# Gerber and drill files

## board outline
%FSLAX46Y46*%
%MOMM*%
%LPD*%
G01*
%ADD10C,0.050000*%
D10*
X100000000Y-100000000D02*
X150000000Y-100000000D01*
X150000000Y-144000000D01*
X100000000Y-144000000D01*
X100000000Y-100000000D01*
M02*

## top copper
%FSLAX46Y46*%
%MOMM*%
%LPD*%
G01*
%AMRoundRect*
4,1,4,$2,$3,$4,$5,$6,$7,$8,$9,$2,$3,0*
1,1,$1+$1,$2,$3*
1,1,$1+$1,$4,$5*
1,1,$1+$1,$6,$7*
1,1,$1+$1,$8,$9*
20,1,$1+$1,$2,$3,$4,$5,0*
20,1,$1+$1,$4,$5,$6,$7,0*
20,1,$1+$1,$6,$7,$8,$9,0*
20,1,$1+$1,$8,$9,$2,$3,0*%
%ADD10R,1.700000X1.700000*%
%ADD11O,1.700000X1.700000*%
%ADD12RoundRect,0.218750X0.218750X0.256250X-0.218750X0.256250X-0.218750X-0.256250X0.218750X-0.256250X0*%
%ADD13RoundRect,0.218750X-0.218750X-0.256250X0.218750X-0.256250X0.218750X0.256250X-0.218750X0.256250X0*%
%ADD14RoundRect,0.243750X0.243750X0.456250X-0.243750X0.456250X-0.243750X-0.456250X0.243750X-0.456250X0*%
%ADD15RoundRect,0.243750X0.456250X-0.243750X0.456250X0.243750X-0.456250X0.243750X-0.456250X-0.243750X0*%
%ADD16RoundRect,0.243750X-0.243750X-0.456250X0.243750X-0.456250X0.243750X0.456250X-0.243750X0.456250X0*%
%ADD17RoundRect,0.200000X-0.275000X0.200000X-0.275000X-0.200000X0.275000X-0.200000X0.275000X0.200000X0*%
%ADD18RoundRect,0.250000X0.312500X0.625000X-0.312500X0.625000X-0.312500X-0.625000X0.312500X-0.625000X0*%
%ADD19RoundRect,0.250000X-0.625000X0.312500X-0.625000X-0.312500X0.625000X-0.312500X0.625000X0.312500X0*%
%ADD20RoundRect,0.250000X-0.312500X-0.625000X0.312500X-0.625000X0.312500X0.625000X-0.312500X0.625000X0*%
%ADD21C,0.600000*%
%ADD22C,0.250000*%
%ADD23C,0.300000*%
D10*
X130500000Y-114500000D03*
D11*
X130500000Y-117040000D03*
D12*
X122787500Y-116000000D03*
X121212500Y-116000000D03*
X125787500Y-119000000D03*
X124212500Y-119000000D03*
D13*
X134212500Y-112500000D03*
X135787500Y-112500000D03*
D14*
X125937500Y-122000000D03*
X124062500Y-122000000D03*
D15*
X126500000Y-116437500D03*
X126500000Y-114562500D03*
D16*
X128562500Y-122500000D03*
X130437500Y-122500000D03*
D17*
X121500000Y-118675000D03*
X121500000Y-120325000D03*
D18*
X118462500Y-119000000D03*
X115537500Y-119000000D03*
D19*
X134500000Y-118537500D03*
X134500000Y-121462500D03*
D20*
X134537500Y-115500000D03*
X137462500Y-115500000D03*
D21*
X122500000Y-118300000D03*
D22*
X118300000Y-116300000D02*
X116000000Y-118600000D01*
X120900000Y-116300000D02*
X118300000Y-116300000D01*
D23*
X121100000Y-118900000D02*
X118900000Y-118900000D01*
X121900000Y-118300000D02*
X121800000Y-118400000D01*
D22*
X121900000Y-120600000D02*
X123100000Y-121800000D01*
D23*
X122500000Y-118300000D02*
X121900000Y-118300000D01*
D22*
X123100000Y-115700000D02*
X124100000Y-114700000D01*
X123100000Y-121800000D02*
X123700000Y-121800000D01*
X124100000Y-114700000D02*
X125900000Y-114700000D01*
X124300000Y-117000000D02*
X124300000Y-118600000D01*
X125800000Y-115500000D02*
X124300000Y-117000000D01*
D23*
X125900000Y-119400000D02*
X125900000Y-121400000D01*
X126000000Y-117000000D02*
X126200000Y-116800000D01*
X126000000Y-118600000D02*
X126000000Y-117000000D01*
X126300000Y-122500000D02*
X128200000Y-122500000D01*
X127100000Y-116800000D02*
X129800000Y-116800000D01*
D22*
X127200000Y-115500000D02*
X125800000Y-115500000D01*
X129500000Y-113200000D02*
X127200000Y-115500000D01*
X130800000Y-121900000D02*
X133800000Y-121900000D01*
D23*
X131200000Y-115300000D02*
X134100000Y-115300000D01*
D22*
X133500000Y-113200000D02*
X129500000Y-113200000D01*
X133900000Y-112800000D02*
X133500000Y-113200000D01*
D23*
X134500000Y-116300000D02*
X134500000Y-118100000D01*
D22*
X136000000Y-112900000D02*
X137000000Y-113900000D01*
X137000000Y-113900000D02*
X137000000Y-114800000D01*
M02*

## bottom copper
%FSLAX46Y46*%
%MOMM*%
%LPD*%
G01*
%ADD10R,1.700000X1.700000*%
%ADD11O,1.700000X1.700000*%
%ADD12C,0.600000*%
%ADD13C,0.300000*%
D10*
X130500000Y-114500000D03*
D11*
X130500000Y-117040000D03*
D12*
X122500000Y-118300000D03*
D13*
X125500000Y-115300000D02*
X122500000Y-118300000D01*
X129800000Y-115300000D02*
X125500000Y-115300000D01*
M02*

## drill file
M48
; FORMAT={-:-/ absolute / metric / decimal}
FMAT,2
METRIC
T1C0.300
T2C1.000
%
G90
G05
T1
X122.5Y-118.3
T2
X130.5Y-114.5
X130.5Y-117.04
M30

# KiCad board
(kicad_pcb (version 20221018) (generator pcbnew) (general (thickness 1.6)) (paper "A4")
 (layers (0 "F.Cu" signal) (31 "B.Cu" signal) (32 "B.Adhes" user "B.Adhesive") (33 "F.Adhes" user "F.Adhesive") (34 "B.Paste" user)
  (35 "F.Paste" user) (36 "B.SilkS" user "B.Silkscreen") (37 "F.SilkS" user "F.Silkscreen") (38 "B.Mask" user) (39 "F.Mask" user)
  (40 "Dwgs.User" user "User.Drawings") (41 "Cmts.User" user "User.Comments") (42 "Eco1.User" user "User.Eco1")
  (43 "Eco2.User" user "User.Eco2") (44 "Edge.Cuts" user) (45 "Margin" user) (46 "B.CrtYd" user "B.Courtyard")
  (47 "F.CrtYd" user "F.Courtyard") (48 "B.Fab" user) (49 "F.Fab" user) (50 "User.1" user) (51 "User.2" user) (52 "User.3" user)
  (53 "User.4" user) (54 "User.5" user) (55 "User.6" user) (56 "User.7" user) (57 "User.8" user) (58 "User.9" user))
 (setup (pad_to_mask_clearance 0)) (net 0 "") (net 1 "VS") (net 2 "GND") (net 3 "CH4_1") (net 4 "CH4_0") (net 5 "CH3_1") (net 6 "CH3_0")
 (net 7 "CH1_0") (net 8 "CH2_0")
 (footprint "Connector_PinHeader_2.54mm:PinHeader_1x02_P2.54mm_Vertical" (layer "F.Cu") (at 130.5 114.5)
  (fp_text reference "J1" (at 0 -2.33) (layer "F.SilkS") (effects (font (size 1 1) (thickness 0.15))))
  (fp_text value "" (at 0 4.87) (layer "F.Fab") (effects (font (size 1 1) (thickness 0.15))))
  (pad "1" thru_hole rect (at 0 0) (size 1.7 1.7) (drill 1) (layers "*.Cu" "*.Mask") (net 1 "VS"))
  (pad "2" thru_hole oval (at 0 2.54) (size 1.7 1.7) (drill 1) (layers "*.Cu" "*.Mask") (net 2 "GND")))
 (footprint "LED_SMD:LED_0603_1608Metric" (layer "F.Cu") (at 122 116 180)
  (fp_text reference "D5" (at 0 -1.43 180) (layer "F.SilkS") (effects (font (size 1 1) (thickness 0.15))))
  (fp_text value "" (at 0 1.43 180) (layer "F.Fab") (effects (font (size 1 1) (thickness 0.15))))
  (pad "1" smd roundrect (at -0.7875 0 180) (size 0.875 0.95) (layers "F.Cu" "F.Paste" "F.Mask") (roundrect_rratio 0.25) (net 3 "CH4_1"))
  (pad "2" smd roundrect (at 0.7875 0 180) (size 0.875 0.95) (layers "F.Cu" "F.Paste" "F.Mask") (roundrect_rratio 0.25) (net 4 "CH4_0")))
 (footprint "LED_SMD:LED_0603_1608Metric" (layer "F.Cu") (at 125 119 180)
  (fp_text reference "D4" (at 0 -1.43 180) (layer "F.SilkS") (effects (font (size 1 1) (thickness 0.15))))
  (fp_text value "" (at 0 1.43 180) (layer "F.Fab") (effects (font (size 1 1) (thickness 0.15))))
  (pad "1" smd roundrect (at -0.7875 0 180) (size 0.875 0.95) (layers "F.Cu" "F.Paste" "F.Mask") (roundrect_rratio 0.25) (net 2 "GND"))
  (pad "2" smd roundrect (at 0.7875 0 180) (size 0.875 0.95) (layers "F.Cu" "F.Paste" "F.Mask") (roundrect_rratio 0.25) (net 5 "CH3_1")))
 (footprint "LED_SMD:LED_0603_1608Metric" (layer "F.Cu") (at 135 112.5)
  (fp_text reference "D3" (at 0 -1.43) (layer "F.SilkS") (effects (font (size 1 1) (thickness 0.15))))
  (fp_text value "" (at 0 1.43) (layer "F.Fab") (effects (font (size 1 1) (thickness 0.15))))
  (pad "1" smd roundrect (at -0.7875 0) (size 0.875 0.95) (layers "F.Cu" "F.Paste" "F.Mask") (roundrect_rratio 0.25) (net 5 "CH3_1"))
  (pad "2" smd roundrect (at 0.7875 0) (size 0.875 0.95) (layers "F.Cu" "F.Paste" "F.Mask") (roundrect_rratio 0.25) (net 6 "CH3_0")))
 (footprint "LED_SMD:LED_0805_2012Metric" (layer "F.Cu") (at 125 122 180)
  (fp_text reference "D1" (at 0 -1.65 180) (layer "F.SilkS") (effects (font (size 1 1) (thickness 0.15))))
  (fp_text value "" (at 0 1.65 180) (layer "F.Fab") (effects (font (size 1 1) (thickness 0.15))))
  (pad "1" smd roundrect (at -0.9375 0 180) (size 0.975 1.4) (layers "F.Cu" "F.Paste" "F.Mask") (roundrect_rratio 0.25) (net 2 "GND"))
  (pad "2" smd roundrect (at 0.9375 0 180) (size 0.975 1.4) (layers "F.Cu" "F.Paste" "F.Mask") (roundrect_rratio 0.25) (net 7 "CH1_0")))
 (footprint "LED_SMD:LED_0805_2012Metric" (layer "F.Cu") (at 126.5 115.5 90)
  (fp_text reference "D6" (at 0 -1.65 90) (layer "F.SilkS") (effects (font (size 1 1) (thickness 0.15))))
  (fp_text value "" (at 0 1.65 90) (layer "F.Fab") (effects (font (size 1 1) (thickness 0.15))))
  (pad "1" smd roundrect (at -0.9375 0 90) (size 0.975 1.4) (layers "F.Cu" "F.Paste" "F.Mask") (roundrect_rratio 0.25) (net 2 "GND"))
  (pad "2" smd roundrect (at 0.9375 0 90) (size 0.975 1.4) (layers "F.Cu" "F.Paste" "F.Mask") (roundrect_rratio 0.25) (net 3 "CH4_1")))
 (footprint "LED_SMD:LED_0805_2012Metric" (layer "F.Cu") (at 129.5 122.5)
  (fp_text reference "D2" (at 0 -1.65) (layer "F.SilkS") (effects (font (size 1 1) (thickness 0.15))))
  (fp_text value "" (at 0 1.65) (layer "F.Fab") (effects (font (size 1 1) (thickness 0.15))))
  (pad "1" smd roundrect (at -0.9375 0) (size 0.975 1.4) (layers "F.Cu" "F.Paste" "F.Mask") (roundrect_rratio 0.25) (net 2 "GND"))
  (pad "2" smd roundrect (at 0.9375 0) (size 0.975 1.4) (layers "F.Cu" "F.Paste" "F.Mask") (roundrect_rratio 0.25) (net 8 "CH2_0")))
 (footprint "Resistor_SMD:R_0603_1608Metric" (layer "F.Cu") (at 121.5 119.5 -90)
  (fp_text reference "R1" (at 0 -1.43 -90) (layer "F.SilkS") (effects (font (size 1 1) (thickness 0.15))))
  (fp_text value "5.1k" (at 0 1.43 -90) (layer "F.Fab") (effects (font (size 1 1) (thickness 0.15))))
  (pad "1" smd roundrect (at -0.825 0 270) (size 0.8 0.95) (layers "F.Cu" "F.Paste" "F.Mask") (roundrect_rratio 0.25) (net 1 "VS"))
  (pad "2" smd roundrect (at 0.825 0 270) (size 0.8 0.95) (layers "F.Cu" "F.Paste" "F.Mask") (roundrect_rratio 0.25) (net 7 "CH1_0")))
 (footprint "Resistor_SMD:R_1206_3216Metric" (layer "F.Cu") (at 117 119 180)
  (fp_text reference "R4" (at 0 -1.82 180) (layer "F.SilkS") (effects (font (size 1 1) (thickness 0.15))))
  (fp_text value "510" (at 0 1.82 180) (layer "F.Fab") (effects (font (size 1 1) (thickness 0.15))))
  (pad "1" smd roundrect (at -1.4625 0 180) (size 1.125 1.75) (layers "F.Cu" "F.Paste" "F.Mask") (roundrect_rratio 0.222222) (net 1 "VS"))
  (pad "2" smd roundrect (at 1.4625 0 180) (size 1.125 1.75) (layers "F.Cu" "F.Paste" "F.Mask") (roundrect_rratio 0.222222) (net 4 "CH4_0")))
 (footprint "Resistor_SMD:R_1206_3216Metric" (layer "F.Cu") (at 134.5 120 -90)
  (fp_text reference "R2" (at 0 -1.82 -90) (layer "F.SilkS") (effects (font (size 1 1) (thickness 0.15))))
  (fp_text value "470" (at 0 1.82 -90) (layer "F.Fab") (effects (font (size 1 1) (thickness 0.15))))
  (pad "1" smd roundrect (at -1.4625 0 270) (size 1.125 1.75) (layers "F.Cu" "F.Paste" "F.Mask") (roundrect_rratio 0.222222) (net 1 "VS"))
  (pad "2" smd roundrect (at 1.4625 0 270) (size 1.125 1.75) (layers "F.Cu" "F.Paste" "F.Mask") (roundrect_rratio 0.222222) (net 8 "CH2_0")))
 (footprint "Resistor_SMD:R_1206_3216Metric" (layer "F.Cu") (at 136 115.5)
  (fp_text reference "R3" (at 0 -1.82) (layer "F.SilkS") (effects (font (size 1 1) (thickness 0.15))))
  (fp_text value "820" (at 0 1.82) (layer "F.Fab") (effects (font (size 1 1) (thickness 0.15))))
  (pad "1" smd roundrect (at -1.4625 0) (size 1.125 1.75) (layers "F.Cu" "F.Paste" "F.Mask") (roundrect_rratio 0.222222) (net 1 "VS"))
  (pad "2" smd roundrect (at 1.4625 0) (size 1.125 1.75) (layers "F.Cu" "F.Paste" "F.Mask") (roundrect_rratio 0.222222) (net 6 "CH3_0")))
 (gr_rect (start 100 100) (end 150 144) (stroke (width 0.05) (type default)) (fill none) (layer "Edge.Cuts"))
 (segment (start 118.3 116.3) (end 116 118.6) (width 0.25) (layer "F.Cu") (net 4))
 (segment (start 120.9 116.3) (end 118.3 116.3) (width 0.25) (layer "F.Cu") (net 4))
 (segment (start 121.1 118.9) (end 118.9 118.9) (width 0.3) (layer "F.Cu") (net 1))
 (segment (start 121.9 118.3) (end 121.8 118.4) (width 0.3) (layer "F.Cu") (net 1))
 (segment (start 121.9 120.6) (end 123.1 121.8) (width 0.25) (layer "F.Cu") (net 7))
 (segment (start 122.5 118.3) (end 121.9 118.3) (width 0.3) (layer "F.Cu") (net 1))
 (segment (start 123.1 115.7) (end 124.1 114.7) (width 0.25) (layer "F.Cu") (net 3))
 (segment (start 123.1 121.8) (end 123.7 121.8) (width 0.25) (layer "F.Cu") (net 7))
 (segment (start 124.1 114.7) (end 125.9 114.7) (width 0.25) (layer "F.Cu") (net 3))
 (segment (start 124.3 117) (end 124.3 118.6) (width 0.25) (layer "F.Cu") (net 5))
 (segment (start 125.8 115.5) (end 124.3 117) (width 0.25) (layer "F.Cu") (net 5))
 (segment (start 125.9 119.4) (end 125.9 121.4) (width 0.3) (layer "F.Cu") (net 2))
 (segment (start 126 117) (end 126.2 116.8) (width 0.3) (layer "F.Cu") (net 2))
 (segment (start 126 118.6) (end 126 117) (width 0.3) (layer "F.Cu") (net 2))
 (segment (start 126.3 122.5) (end 128.2 122.5) (width 0.3) (layer "F.Cu") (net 2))
 (segment (start 127.1 116.8) (end 129.8 116.8) (width 0.3) (layer "F.Cu") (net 2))
 (segment (start 127.2 115.5) (end 125.8 115.5) (width 0.25) (layer "F.Cu") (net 5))
 (segment (start 129.5 113.2) (end 127.2 115.5) (width 0.25) (layer "F.Cu") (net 5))
 (segment (start 130.8 121.9) (end 133.8 121.9) (width 0.25) (layer "F.Cu") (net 8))
 (segment (start 131.2 115.3) (end 134.1 115.3) (width 0.3) (layer "F.Cu") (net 1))
 (segment (start 133.5 113.2) (end 129.5 113.2) (width 0.25) (layer "F.Cu") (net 5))
 (segment (start 133.9 112.8) (end 133.5 113.2) (width 0.25) (layer "F.Cu") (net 5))
 (segment (start 134.5 116.3) (end 134.5 118.1) (width 0.3) (layer "F.Cu") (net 1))
 (segment (start 136 112.9) (end 137 113.9) (width 0.25) (layer "F.Cu") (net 6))
 (segment (start 137 113.9) (end 137 114.8) (width 0.25) (layer "F.Cu") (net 6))
 (via (at 122.5 118.3) (size 0.6) (drill 0.3) (layers "F.Cu" "B.Cu") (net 1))
 (segment (start 125.5 115.3) (end 122.5 118.3) (width 0.3) (layer "B.Cu") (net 1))
 (segment (start 129.8 115.3) (end 125.5 115.3) (width 0.3) (layer "B.Cu") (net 1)))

